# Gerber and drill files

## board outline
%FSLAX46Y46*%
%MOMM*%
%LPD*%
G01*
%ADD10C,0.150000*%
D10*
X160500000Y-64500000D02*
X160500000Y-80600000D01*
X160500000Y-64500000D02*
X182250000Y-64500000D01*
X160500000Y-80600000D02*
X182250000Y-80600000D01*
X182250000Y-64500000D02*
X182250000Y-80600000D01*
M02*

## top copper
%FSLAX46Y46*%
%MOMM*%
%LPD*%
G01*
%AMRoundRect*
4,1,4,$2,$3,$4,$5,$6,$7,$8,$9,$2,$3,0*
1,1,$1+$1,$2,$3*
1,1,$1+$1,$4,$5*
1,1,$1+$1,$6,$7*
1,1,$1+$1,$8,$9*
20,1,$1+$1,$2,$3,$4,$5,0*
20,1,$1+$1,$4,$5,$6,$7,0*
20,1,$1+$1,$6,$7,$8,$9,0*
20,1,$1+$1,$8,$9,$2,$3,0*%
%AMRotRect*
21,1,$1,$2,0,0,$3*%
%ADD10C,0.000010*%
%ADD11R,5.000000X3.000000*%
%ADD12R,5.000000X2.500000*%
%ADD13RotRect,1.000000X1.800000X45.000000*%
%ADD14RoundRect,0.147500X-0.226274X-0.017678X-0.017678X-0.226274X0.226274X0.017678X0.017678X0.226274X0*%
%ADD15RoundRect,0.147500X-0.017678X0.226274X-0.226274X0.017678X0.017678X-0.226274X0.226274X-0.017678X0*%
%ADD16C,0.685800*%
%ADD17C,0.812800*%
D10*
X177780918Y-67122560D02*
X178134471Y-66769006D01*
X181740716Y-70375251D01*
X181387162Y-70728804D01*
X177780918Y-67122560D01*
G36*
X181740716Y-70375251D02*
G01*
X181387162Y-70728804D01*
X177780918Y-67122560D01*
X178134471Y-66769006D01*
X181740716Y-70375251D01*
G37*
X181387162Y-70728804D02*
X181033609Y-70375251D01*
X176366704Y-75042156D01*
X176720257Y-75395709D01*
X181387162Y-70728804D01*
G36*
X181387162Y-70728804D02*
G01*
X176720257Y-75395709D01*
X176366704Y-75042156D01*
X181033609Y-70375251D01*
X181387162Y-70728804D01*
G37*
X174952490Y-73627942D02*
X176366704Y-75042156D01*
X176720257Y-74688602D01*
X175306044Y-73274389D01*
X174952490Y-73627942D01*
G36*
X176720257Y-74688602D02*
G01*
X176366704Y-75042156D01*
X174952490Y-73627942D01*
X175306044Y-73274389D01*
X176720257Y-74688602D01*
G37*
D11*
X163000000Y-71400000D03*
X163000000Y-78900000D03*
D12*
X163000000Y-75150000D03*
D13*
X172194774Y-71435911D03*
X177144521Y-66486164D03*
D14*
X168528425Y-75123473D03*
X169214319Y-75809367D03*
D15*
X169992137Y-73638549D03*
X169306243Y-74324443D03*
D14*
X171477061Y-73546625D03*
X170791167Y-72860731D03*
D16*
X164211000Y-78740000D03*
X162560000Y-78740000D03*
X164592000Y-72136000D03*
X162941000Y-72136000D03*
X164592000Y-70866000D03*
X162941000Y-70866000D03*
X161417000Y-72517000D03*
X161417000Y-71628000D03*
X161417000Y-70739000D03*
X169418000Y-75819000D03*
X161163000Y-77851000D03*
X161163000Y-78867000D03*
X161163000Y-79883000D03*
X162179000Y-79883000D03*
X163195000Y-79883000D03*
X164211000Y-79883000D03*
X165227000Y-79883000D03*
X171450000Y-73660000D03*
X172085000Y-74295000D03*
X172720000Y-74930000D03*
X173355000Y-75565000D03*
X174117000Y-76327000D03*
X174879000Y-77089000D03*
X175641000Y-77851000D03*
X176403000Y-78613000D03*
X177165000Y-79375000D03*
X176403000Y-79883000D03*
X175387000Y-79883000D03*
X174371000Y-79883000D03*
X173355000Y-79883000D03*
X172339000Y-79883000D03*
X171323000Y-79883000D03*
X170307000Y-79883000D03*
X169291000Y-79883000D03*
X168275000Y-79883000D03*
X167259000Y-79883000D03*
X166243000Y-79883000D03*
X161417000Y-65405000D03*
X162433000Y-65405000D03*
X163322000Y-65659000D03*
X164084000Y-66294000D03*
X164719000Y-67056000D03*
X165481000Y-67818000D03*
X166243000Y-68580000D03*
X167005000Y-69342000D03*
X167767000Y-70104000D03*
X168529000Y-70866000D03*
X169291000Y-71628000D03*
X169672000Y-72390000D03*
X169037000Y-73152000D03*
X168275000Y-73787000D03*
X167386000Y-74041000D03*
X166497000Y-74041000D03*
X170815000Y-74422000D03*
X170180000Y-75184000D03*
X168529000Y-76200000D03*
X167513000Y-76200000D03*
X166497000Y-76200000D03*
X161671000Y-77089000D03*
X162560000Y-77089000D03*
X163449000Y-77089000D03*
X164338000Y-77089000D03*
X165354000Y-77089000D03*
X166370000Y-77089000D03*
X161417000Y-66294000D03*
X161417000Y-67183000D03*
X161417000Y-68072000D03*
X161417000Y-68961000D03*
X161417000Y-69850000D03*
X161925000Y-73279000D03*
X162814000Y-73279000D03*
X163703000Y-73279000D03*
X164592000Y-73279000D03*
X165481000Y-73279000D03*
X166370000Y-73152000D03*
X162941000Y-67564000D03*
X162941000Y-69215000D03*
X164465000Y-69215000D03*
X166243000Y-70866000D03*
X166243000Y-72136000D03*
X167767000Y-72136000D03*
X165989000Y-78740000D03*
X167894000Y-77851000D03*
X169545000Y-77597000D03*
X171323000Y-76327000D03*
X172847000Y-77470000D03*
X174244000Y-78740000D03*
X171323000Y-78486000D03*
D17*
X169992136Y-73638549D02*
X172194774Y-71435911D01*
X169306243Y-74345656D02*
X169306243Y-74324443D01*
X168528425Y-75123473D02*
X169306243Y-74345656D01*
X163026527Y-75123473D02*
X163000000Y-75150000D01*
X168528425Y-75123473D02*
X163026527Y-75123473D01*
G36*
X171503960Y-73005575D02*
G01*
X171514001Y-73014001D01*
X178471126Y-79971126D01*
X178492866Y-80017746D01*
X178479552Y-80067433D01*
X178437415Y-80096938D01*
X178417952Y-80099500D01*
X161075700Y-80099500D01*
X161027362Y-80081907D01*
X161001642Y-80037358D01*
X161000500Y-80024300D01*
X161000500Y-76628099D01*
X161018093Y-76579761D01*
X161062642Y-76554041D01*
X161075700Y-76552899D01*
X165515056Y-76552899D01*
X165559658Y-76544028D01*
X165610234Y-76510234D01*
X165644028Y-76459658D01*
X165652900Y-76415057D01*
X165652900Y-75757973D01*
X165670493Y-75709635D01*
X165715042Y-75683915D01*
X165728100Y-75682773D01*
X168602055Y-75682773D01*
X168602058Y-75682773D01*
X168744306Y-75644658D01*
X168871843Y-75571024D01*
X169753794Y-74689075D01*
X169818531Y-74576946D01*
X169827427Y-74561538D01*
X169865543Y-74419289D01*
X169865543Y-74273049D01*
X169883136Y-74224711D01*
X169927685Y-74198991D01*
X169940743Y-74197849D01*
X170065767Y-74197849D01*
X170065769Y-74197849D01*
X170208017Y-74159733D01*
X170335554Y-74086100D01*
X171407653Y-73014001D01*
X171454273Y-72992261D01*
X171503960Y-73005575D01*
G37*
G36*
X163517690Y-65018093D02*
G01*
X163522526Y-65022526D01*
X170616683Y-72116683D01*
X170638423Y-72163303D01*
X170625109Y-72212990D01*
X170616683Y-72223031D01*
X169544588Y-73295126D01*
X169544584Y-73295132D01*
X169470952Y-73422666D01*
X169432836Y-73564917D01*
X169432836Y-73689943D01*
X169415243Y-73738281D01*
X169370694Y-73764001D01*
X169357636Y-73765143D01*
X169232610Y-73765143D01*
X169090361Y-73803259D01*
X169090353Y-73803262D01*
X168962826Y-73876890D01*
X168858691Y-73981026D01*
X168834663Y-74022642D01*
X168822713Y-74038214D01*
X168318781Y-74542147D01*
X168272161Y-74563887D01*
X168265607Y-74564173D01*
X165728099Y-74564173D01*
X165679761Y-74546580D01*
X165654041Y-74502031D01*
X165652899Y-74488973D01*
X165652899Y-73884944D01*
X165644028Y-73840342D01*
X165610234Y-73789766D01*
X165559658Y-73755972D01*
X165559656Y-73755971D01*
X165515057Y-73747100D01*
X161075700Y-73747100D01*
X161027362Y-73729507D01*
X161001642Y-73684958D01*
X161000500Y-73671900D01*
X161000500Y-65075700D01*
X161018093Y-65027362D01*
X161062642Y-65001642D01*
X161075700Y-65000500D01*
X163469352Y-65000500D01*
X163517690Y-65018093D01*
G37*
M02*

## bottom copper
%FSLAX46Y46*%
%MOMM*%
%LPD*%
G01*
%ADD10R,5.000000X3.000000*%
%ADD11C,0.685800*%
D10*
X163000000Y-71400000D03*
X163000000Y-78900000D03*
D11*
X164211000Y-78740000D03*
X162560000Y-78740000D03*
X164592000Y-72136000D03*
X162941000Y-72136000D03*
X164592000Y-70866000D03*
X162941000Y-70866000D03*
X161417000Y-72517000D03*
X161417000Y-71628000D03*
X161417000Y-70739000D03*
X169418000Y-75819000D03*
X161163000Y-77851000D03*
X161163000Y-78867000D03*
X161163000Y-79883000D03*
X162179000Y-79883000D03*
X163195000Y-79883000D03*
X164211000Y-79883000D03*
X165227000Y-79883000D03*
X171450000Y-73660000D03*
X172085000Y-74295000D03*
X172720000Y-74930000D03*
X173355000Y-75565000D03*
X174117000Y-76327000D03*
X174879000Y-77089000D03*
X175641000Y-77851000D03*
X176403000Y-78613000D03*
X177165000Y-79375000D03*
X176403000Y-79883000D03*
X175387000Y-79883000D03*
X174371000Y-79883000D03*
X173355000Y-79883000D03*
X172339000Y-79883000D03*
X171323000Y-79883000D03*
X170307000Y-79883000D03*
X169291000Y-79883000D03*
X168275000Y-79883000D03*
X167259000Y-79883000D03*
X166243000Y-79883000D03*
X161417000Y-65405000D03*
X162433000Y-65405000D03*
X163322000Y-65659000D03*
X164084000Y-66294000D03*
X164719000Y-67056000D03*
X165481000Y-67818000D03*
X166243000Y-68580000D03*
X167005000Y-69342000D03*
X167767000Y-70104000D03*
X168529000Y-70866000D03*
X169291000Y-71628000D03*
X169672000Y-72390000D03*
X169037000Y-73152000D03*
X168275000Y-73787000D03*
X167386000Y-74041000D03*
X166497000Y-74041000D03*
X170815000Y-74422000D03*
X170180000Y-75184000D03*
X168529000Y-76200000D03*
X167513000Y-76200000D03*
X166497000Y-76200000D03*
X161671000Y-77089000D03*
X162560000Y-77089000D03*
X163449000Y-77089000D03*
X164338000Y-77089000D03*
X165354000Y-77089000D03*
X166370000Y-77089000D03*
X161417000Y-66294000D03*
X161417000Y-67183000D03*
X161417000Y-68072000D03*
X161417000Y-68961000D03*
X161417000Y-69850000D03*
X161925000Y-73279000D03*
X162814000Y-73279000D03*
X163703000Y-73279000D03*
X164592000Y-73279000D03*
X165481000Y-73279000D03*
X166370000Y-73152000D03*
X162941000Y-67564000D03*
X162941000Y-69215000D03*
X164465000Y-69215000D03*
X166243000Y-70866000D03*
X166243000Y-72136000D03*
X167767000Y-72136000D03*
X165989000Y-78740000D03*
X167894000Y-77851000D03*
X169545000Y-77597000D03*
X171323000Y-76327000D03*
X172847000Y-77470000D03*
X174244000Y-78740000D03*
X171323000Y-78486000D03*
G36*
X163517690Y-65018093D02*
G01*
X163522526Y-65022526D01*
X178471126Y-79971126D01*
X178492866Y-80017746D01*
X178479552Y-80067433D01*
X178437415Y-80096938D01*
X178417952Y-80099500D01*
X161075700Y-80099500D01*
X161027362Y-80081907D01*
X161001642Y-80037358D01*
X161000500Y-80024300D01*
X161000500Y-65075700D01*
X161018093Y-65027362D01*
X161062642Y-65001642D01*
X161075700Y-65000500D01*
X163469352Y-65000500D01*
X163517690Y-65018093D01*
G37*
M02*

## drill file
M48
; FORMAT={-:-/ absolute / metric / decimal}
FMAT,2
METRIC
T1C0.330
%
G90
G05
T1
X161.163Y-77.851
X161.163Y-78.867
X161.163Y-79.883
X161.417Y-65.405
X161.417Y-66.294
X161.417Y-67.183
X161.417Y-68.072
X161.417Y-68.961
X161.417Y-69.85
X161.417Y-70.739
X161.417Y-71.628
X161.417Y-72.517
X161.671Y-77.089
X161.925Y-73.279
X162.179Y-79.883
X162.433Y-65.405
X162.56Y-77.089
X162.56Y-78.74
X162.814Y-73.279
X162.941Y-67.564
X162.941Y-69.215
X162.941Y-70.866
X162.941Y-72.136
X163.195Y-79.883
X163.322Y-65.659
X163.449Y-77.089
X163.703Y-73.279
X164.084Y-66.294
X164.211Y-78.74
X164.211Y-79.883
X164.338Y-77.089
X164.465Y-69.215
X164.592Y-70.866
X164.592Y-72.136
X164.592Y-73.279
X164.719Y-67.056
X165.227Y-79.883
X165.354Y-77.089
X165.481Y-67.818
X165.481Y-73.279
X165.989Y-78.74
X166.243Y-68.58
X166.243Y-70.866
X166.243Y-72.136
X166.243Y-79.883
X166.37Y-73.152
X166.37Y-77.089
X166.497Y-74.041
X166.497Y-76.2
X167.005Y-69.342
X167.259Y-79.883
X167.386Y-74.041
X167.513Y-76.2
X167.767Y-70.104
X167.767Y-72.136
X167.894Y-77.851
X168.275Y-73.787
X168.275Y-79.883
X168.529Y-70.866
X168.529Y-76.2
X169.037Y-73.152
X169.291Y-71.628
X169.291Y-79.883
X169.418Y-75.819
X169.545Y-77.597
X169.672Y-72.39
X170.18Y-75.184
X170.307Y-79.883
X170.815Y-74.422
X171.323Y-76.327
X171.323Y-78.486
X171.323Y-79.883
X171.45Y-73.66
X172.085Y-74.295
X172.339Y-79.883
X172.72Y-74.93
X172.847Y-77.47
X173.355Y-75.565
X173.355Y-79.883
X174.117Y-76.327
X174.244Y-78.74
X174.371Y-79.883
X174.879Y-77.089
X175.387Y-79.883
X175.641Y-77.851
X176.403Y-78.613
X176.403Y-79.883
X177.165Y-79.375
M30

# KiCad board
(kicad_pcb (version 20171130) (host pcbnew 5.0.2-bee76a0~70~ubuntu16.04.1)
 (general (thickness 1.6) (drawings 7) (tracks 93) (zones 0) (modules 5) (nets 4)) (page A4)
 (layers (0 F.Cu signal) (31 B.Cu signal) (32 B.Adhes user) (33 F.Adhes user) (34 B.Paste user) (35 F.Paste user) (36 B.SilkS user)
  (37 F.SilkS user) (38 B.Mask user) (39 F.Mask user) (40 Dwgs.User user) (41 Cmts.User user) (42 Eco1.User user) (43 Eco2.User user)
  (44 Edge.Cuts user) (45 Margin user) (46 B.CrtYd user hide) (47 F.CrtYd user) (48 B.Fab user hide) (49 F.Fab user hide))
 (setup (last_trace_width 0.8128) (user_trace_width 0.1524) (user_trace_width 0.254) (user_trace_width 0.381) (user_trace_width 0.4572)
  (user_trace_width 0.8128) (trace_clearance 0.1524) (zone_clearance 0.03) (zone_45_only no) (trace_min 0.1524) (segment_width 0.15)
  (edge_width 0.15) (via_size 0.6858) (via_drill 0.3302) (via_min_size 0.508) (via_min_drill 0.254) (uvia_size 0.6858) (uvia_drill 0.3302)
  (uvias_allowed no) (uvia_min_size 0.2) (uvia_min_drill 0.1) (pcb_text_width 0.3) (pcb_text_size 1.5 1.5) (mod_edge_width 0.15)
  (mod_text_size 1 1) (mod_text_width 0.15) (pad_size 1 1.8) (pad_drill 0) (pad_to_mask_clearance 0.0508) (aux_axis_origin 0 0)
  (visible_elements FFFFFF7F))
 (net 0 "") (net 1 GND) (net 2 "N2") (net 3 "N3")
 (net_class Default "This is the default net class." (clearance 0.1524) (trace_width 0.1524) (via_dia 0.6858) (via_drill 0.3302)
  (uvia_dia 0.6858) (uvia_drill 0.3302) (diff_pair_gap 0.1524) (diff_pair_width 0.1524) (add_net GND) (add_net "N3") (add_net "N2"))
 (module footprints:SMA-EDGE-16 (layer F.Cu) (at 163 69.9 180)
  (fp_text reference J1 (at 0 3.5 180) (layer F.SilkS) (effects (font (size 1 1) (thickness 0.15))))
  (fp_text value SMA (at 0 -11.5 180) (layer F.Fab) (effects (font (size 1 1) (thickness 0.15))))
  (pad 1 smd rect (at 0 -1.5 180) (size 5 3) (layers F.Cu F.Paste F.Mask) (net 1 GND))
  (pad 2 smd rect (at 0 -7.5 180) (size 5 3) (drill (offset 0 -1.5)) (layers F.Cu F.Paste F.Mask) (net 1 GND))
  (pad 3 smd rect (at 0 0 180) (size 5 3) (drill (offset 0 -1.5)) (layers B.Cu B.Paste B.Mask) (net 1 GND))
  (pad 4 smd rect (at 0 -7.5 180) (size 5 3) (drill (offset 0 -1.5)) (layers B.Cu B.Paste B.Mask) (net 1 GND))
  (pad 5 smd rect (at 0 -5.25 180) (size 5 2.5) (layers F.Cu F.Paste F.Mask) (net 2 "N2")))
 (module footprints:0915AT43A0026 (layer F.Cu) (at 172.194774 71.435911 45)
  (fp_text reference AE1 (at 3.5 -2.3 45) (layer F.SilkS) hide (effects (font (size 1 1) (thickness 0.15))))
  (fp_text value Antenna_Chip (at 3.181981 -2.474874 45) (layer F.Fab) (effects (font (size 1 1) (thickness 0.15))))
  (fp_poly (pts (xy 7 0.9) (xy 7.5 0.9) (xy 7.5 6) (xy 7 6)) (layer F.Cu) (width 0.00001))
  (fp_poly (pts (xy 7 6) (xy 7 5.5) (xy 0.4 5.5) (xy 0.4 6)) (layer F.Cu) (width 0.00001))
  (fp_poly (pts (xy 0.4 3.5) (xy 0.4 5.5) (xy 0.9 5.5) (xy 0.9 3.5)) (layer F.Cu) (width 0.00001))
  (pad 1 smd rect (at 0 0 45) (size 1 1.8) (layers F.Cu F.Paste F.Mask) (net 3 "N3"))
  (pad 2 smd rect (at 7 0 45) (size 1 1.8) (layers F.Cu F.Paste F.Mask)))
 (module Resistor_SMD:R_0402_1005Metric (layer F.Cu) (at 168.871372 75.46642 315)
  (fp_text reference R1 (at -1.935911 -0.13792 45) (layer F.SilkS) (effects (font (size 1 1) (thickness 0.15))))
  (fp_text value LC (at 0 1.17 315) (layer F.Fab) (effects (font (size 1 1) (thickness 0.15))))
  (pad 1 smd roundrect (at -0.485 0 315) (size 0.59 0.64) (layers F.Cu F.Paste F.Mask) (roundrect_rratio 0.25) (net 2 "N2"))
  (pad 2 smd roundrect (at 0.485 0 315) (size 0.59 0.64) (layers F.Cu F.Paste F.Mask) (roundrect_rratio 0.25) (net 1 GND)))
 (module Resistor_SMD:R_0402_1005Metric (layer F.Cu) (at 169.64919 73.981496 225)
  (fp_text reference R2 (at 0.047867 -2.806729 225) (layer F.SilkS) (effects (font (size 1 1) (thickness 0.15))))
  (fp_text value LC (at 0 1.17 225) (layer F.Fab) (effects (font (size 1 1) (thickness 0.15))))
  (pad 1 smd roundrect (at -0.485 0 225) (size 0.59 0.64) (layers F.Cu F.Paste F.Mask) (roundrect_rratio 0.25) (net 3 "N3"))
  (pad 2 smd roundrect (at 0.485 0 225) (size 0.59 0.64) (layers F.Cu F.Paste F.Mask) (roundrect_rratio 0.25) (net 2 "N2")))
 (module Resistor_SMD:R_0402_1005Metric (layer F.Cu) (at 171.134114 73.203678 315)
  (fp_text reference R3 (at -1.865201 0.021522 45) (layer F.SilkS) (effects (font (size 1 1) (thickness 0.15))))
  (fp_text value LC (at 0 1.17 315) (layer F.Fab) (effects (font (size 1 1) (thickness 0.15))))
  (pad 2 smd roundrect (at 0.485 0 315) (size 0.59 0.64) (layers F.Cu F.Paste F.Mask) (roundrect_rratio 0.25) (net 1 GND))
  (pad 1 smd roundrect (at -0.485 0 315) (size 0.59 0.64) (layers F.Cu F.Paste F.Mask) (roundrect_rratio 0.25) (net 3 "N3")))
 (gr_line (start 160.5 64.5) (end 160.5 80.6) (layer Edge.Cuts) (width 0.15))
 (gr_line (start 160.5 64.5) (end 182.25 64.5) (layer Edge.Cuts) (width 0.15))
 (gr_line (start 160.5 80.6) (end 182.25 80.6) (layer Edge.Cuts) (width 0.15))
 (gr_line (start 182.25 64.5) (end 182.25 80.6) (layer Edge.Cuts) (width 0.15))
 (via (at 164.211 78.74) (size 0.6858) (drill 0.3302) (layers F.Cu B.Cu) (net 1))
 (via (at 162.56 78.74) (size 0.6858) (drill 0.3302) (layers F.Cu B.Cu) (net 1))
 (via (at 164.592 72.136) (size 0.6858) (drill 0.3302) (layers F.Cu B.Cu) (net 1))
 (via (at 162.941 72.136) (size 0.6858) (drill 0.3302) (layers F.Cu B.Cu) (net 1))
 (via (at 164.592 70.866) (size 0.6858) (drill 0.3302) (layers F.Cu B.Cu) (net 1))
 (via (at 162.941 70.866) (size 0.6858) (drill 0.3302) (layers F.Cu B.Cu) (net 1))
 (via (at 161.417 72.517) (size 0.6858) (drill 0.3302) (layers F.Cu B.Cu) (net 1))
 (via (at 161.417 71.628) (size 0.6858) (drill 0.3302) (layers F.Cu B.Cu) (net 1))
 (via (at 161.417 70.739) (size 0.6858) (drill 0.3302) (layers F.Cu B.Cu) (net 1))
 (via (at 169.418 75.819) (size 0.6858) (drill 0.3302) (layers F.Cu B.Cu) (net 1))
 (via (at 161.163 77.851) (size 0.6858) (drill 0.3302) (layers F.Cu B.Cu) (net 1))
 (via (at 161.163 78.867) (size 0.6858) (drill 0.3302) (layers F.Cu B.Cu) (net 1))
 (via (at 161.163 79.883) (size 0.6858) (drill 0.3302) (layers F.Cu B.Cu) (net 1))
 (via (at 162.179 79.883) (size 0.6858) (drill 0.3302) (layers F.Cu B.Cu) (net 1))
 (via (at 163.195 79.883) (size 0.6858) (drill 0.3302) (layers F.Cu B.Cu) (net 1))
 (via (at 164.211 79.883) (size 0.6858) (drill 0.3302) (layers F.Cu B.Cu) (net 1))
 (via (at 165.227 79.883) (size 0.6858) (drill 0.3302) (layers F.Cu B.Cu) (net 1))
 (segment (start 169.992136 73.638549) (end 172.194774 71.435911) (width 0.8128) (layer F.Cu) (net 3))
 (segment (start 169.306243 74.345656) (end 169.306243 74.324443) (width 0.8128) (layer F.Cu) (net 2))
 (segment (start 168.528425 75.123473) (end 169.306243 74.345656) (width 0.8128) (layer F.Cu) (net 2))
 (segment (start 163.026527 75.123473) (end 163 75.15) (width 0.8128) (layer F.Cu) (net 2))
 (segment (start 168.528425 75.123473) (end 163.026527 75.123473) (width 0.8128) (layer F.Cu) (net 2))
 (via (at 171.45 73.66) (size 0.6858) (drill 0.3302) (layers F.Cu B.Cu) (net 1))
 (via (at 172.085 74.295) (size 0.6858) (drill 0.3302) (layers F.Cu B.Cu) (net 1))
 (via (at 172.72 74.93) (size 0.6858) (drill 0.3302) (layers F.Cu B.Cu) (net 1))
 (via (at 173.355 75.565) (size 0.6858) (drill 0.3302) (layers F.Cu B.Cu) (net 1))
 (via (at 174.117 76.327) (size 0.6858) (drill 0.3302) (layers F.Cu B.Cu) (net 1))
 (via (at 174.879 77.089) (size 0.6858) (drill 0.3302) (layers F.Cu B.Cu) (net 1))
 (via (at 175.641 77.851) (size 0.6858) (drill 0.3302) (layers F.Cu B.Cu) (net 1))
 (via (at 176.403 78.613) (size 0.6858) (drill 0.3302) (layers F.Cu B.Cu) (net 1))
 (via (at 177.165 79.375) (size 0.6858) (drill 0.3302) (layers F.Cu B.Cu) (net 1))
 (via (at 176.403 79.883) (size 0.6858) (drill 0.3302) (layers F.Cu B.Cu) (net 1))
 (via (at 175.387 79.883) (size 0.6858) (drill 0.3302) (layers F.Cu B.Cu) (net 1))
 (via (at 174.371 79.883) (size 0.6858) (drill 0.3302) (layers F.Cu B.Cu) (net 1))
 (via (at 173.355 79.883) (size 0.6858) (drill 0.3302) (layers F.Cu B.Cu) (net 1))
 (via (at 172.339 79.883) (size 0.6858) (drill 0.3302) (layers F.Cu B.Cu) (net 1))
 (via (at 171.323 79.883) (size 0.6858) (drill 0.3302) (layers F.Cu B.Cu) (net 1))
 (via (at 170.307 79.883) (size 0.6858) (drill 0.3302) (layers F.Cu B.Cu) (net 1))
 (via (at 169.291 79.883) (size 0.6858) (drill 0.3302) (layers F.Cu B.Cu) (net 1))
 (via (at 168.275 79.883) (size 0.6858) (drill 0.3302) (layers F.Cu B.Cu) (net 1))
 (via (at 167.259 79.883) (size 0.6858) (drill 0.3302) (layers F.Cu B.Cu) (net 1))
 (via (at 166.243 79.883) (size 0.6858) (drill 0.3302) (layers F.Cu B.Cu) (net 1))
 (via (at 161.417 65.405) (size 0.6858) (drill 0.3302) (layers F.Cu B.Cu) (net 1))
 (via (at 162.433 65.405) (size 0.6858) (drill 0.3302) (layers F.Cu B.Cu) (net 1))
 (via (at 163.322 65.659) (size 0.6858) (drill 0.3302) (layers F.Cu B.Cu) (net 1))
 (via (at 164.084 66.294) (size 0.6858) (drill 0.3302) (layers F.Cu B.Cu) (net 1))
 (via (at 164.719 67.056) (size 0.6858) (drill 0.3302) (layers F.Cu B.Cu) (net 1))
 (via (at 165.481 67.818) (size 0.6858) (drill 0.3302) (layers F.Cu B.Cu) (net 1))
 (via (at 166.243 68.58) (size 0.6858) (drill 0.3302) (layers F.Cu B.Cu) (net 1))
 (via (at 167.005 69.342) (size 0.6858) (drill 0.3302) (layers F.Cu B.Cu) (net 1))
 (via (at 167.767 70.104) (size 0.6858) (drill 0.3302) (layers F.Cu B.Cu) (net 1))
 (via (at 168.529 70.866) (size 0.6858) (drill 0.3302) (layers F.Cu B.Cu) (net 1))
 (via (at 169.291 71.628) (size 0.6858) (drill 0.3302) (layers F.Cu B.Cu) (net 1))
 (via (at 169.672 72.39) (size 0.6858) (drill 0.3302) (layers F.Cu B.Cu) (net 1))
 (via (at 169.037 73.152) (size 0.6858) (drill 0.3302) (layers F.Cu B.Cu) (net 1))
 (via (at 168.275 73.787) (size 0.6858) (drill 0.3302) (layers F.Cu B.Cu) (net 1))
 (via (at 167.386 74.041) (size 0.6858) (drill 0.3302) (layers F.Cu B.Cu) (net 1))
 (via (at 166.497 74.041) (size 0.6858) (drill 0.3302) (layers F.Cu B.Cu) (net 1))
 (via (at 170.815 74.422) (size 0.6858) (drill 0.3302) (layers F.Cu B.Cu) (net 1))
 (via (at 170.18 75.184) (size 0.6858) (drill 0.3302) (layers F.Cu B.Cu) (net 1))
 (via (at 168.529 76.2) (size 0.6858) (drill 0.3302) (layers F.Cu B.Cu) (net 1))
 (via (at 167.513 76.2) (size 0.6858) (drill 0.3302) (layers F.Cu B.Cu) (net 1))
 (via (at 166.497 76.2) (size 0.6858) (drill 0.3302) (layers F.Cu B.Cu) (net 1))
 (via (at 161.671 77.089) (size 0.6858) (drill 0.3302) (layers F.Cu B.Cu) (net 1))
 (via (at 162.56 77.089) (size 0.6858) (drill 0.3302) (layers F.Cu B.Cu) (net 1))
 (via (at 163.449 77.089) (size 0.6858) (drill 0.3302) (layers F.Cu B.Cu) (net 1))
 (via (at 164.338 77.089) (size 0.6858) (drill 0.3302) (layers F.Cu B.Cu) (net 1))
 (via (at 165.354 77.089) (size 0.6858) (drill 0.3302) (layers F.Cu B.Cu) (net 1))
 (via (at 166.37 77.089) (size 0.6858) (drill 0.3302) (layers F.Cu B.Cu) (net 1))
 (via (at 161.417 66.294) (size 0.6858) (drill 0.3302) (layers F.Cu B.Cu) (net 1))
 (via (at 161.417 67.183) (size 0.6858) (drill 0.3302) (layers F.Cu B.Cu) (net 1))
 (via (at 161.417 68.072) (size 0.6858) (drill 0.3302) (layers F.Cu B.Cu) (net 1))
 (via (at 161.417 68.961) (size 0.6858) (drill 0.3302) (layers F.Cu B.Cu) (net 1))
 (via (at 161.417 69.85) (size 0.6858) (drill 0.3302) (layers F.Cu B.Cu) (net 1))
 (via (at 161.925 73.279) (size 0.6858) (drill 0.3302) (layers F.Cu B.Cu) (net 1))
 (via (at 162.814 73.279) (size 0.6858) (drill 0.3302) (layers F.Cu B.Cu) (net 1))
 (via (at 163.703 73.279) (size 0.6858) (drill 0.3302) (layers F.Cu B.Cu) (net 1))
 (via (at 164.592 73.279) (size 0.6858) (drill 0.3302) (layers F.Cu B.Cu) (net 1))
 (via (at 165.481 73.279) (size 0.6858) (drill 0.3302) (layers F.Cu B.Cu) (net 1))
 (via (at 166.37 73.152) (size 0.6858) (drill 0.3302) (layers F.Cu B.Cu) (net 1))
 (via (at 162.941 67.564) (size 0.6858) (drill 0.3302) (layers F.Cu B.Cu) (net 1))
 (via (at 162.941 69.215) (size 0.6858) (drill 0.3302) (layers F.Cu B.Cu) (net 1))
 (via (at 164.465 69.215) (size 0.6858) (drill 0.3302) (layers F.Cu B.Cu) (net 1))
 (via (at 166.243 70.866) (size 0.6858) (drill 0.3302) (layers F.Cu B.Cu) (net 1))
 (via (at 166.243 72.136) (size 0.6858) (drill 0.3302) (layers F.Cu B.Cu) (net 1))
 (via (at 167.767 72.136) (size 0.6858) (drill 0.3302) (layers F.Cu B.Cu) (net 1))
 (via (at 165.989 78.74) (size 0.6858) (drill 0.3302) (layers F.Cu B.Cu) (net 1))
 (via (at 167.894 77.851) (size 0.6858) (drill 0.3302) (layers F.Cu B.Cu) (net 1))
 (via (at 169.545 77.597) (size 0.6858) (drill 0.3302) (layers F.Cu B.Cu) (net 1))
 (via (at 171.323 76.327) (size 0.6858) (drill 0.3302) (layers F.Cu B.Cu) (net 1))
 (via (at 172.847 77.47) (size 0.6858) (drill 0.3302) (layers F.Cu B.Cu) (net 1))
 (via (at 174.244 78.74) (size 0.6858) (drill 0.3302) (layers F.Cu B.Cu) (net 1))
 (via (at 171.323 78.486) (size 0.6858) (drill 0.3302) (layers F.Cu B.Cu) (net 1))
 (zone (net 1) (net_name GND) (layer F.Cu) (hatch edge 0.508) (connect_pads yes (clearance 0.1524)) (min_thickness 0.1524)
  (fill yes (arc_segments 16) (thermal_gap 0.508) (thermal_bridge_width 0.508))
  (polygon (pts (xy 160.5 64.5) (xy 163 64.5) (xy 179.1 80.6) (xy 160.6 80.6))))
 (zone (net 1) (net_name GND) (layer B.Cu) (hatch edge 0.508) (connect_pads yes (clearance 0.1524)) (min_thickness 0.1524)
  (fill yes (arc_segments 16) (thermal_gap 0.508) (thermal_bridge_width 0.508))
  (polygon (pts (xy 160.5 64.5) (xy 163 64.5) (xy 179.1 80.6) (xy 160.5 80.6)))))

